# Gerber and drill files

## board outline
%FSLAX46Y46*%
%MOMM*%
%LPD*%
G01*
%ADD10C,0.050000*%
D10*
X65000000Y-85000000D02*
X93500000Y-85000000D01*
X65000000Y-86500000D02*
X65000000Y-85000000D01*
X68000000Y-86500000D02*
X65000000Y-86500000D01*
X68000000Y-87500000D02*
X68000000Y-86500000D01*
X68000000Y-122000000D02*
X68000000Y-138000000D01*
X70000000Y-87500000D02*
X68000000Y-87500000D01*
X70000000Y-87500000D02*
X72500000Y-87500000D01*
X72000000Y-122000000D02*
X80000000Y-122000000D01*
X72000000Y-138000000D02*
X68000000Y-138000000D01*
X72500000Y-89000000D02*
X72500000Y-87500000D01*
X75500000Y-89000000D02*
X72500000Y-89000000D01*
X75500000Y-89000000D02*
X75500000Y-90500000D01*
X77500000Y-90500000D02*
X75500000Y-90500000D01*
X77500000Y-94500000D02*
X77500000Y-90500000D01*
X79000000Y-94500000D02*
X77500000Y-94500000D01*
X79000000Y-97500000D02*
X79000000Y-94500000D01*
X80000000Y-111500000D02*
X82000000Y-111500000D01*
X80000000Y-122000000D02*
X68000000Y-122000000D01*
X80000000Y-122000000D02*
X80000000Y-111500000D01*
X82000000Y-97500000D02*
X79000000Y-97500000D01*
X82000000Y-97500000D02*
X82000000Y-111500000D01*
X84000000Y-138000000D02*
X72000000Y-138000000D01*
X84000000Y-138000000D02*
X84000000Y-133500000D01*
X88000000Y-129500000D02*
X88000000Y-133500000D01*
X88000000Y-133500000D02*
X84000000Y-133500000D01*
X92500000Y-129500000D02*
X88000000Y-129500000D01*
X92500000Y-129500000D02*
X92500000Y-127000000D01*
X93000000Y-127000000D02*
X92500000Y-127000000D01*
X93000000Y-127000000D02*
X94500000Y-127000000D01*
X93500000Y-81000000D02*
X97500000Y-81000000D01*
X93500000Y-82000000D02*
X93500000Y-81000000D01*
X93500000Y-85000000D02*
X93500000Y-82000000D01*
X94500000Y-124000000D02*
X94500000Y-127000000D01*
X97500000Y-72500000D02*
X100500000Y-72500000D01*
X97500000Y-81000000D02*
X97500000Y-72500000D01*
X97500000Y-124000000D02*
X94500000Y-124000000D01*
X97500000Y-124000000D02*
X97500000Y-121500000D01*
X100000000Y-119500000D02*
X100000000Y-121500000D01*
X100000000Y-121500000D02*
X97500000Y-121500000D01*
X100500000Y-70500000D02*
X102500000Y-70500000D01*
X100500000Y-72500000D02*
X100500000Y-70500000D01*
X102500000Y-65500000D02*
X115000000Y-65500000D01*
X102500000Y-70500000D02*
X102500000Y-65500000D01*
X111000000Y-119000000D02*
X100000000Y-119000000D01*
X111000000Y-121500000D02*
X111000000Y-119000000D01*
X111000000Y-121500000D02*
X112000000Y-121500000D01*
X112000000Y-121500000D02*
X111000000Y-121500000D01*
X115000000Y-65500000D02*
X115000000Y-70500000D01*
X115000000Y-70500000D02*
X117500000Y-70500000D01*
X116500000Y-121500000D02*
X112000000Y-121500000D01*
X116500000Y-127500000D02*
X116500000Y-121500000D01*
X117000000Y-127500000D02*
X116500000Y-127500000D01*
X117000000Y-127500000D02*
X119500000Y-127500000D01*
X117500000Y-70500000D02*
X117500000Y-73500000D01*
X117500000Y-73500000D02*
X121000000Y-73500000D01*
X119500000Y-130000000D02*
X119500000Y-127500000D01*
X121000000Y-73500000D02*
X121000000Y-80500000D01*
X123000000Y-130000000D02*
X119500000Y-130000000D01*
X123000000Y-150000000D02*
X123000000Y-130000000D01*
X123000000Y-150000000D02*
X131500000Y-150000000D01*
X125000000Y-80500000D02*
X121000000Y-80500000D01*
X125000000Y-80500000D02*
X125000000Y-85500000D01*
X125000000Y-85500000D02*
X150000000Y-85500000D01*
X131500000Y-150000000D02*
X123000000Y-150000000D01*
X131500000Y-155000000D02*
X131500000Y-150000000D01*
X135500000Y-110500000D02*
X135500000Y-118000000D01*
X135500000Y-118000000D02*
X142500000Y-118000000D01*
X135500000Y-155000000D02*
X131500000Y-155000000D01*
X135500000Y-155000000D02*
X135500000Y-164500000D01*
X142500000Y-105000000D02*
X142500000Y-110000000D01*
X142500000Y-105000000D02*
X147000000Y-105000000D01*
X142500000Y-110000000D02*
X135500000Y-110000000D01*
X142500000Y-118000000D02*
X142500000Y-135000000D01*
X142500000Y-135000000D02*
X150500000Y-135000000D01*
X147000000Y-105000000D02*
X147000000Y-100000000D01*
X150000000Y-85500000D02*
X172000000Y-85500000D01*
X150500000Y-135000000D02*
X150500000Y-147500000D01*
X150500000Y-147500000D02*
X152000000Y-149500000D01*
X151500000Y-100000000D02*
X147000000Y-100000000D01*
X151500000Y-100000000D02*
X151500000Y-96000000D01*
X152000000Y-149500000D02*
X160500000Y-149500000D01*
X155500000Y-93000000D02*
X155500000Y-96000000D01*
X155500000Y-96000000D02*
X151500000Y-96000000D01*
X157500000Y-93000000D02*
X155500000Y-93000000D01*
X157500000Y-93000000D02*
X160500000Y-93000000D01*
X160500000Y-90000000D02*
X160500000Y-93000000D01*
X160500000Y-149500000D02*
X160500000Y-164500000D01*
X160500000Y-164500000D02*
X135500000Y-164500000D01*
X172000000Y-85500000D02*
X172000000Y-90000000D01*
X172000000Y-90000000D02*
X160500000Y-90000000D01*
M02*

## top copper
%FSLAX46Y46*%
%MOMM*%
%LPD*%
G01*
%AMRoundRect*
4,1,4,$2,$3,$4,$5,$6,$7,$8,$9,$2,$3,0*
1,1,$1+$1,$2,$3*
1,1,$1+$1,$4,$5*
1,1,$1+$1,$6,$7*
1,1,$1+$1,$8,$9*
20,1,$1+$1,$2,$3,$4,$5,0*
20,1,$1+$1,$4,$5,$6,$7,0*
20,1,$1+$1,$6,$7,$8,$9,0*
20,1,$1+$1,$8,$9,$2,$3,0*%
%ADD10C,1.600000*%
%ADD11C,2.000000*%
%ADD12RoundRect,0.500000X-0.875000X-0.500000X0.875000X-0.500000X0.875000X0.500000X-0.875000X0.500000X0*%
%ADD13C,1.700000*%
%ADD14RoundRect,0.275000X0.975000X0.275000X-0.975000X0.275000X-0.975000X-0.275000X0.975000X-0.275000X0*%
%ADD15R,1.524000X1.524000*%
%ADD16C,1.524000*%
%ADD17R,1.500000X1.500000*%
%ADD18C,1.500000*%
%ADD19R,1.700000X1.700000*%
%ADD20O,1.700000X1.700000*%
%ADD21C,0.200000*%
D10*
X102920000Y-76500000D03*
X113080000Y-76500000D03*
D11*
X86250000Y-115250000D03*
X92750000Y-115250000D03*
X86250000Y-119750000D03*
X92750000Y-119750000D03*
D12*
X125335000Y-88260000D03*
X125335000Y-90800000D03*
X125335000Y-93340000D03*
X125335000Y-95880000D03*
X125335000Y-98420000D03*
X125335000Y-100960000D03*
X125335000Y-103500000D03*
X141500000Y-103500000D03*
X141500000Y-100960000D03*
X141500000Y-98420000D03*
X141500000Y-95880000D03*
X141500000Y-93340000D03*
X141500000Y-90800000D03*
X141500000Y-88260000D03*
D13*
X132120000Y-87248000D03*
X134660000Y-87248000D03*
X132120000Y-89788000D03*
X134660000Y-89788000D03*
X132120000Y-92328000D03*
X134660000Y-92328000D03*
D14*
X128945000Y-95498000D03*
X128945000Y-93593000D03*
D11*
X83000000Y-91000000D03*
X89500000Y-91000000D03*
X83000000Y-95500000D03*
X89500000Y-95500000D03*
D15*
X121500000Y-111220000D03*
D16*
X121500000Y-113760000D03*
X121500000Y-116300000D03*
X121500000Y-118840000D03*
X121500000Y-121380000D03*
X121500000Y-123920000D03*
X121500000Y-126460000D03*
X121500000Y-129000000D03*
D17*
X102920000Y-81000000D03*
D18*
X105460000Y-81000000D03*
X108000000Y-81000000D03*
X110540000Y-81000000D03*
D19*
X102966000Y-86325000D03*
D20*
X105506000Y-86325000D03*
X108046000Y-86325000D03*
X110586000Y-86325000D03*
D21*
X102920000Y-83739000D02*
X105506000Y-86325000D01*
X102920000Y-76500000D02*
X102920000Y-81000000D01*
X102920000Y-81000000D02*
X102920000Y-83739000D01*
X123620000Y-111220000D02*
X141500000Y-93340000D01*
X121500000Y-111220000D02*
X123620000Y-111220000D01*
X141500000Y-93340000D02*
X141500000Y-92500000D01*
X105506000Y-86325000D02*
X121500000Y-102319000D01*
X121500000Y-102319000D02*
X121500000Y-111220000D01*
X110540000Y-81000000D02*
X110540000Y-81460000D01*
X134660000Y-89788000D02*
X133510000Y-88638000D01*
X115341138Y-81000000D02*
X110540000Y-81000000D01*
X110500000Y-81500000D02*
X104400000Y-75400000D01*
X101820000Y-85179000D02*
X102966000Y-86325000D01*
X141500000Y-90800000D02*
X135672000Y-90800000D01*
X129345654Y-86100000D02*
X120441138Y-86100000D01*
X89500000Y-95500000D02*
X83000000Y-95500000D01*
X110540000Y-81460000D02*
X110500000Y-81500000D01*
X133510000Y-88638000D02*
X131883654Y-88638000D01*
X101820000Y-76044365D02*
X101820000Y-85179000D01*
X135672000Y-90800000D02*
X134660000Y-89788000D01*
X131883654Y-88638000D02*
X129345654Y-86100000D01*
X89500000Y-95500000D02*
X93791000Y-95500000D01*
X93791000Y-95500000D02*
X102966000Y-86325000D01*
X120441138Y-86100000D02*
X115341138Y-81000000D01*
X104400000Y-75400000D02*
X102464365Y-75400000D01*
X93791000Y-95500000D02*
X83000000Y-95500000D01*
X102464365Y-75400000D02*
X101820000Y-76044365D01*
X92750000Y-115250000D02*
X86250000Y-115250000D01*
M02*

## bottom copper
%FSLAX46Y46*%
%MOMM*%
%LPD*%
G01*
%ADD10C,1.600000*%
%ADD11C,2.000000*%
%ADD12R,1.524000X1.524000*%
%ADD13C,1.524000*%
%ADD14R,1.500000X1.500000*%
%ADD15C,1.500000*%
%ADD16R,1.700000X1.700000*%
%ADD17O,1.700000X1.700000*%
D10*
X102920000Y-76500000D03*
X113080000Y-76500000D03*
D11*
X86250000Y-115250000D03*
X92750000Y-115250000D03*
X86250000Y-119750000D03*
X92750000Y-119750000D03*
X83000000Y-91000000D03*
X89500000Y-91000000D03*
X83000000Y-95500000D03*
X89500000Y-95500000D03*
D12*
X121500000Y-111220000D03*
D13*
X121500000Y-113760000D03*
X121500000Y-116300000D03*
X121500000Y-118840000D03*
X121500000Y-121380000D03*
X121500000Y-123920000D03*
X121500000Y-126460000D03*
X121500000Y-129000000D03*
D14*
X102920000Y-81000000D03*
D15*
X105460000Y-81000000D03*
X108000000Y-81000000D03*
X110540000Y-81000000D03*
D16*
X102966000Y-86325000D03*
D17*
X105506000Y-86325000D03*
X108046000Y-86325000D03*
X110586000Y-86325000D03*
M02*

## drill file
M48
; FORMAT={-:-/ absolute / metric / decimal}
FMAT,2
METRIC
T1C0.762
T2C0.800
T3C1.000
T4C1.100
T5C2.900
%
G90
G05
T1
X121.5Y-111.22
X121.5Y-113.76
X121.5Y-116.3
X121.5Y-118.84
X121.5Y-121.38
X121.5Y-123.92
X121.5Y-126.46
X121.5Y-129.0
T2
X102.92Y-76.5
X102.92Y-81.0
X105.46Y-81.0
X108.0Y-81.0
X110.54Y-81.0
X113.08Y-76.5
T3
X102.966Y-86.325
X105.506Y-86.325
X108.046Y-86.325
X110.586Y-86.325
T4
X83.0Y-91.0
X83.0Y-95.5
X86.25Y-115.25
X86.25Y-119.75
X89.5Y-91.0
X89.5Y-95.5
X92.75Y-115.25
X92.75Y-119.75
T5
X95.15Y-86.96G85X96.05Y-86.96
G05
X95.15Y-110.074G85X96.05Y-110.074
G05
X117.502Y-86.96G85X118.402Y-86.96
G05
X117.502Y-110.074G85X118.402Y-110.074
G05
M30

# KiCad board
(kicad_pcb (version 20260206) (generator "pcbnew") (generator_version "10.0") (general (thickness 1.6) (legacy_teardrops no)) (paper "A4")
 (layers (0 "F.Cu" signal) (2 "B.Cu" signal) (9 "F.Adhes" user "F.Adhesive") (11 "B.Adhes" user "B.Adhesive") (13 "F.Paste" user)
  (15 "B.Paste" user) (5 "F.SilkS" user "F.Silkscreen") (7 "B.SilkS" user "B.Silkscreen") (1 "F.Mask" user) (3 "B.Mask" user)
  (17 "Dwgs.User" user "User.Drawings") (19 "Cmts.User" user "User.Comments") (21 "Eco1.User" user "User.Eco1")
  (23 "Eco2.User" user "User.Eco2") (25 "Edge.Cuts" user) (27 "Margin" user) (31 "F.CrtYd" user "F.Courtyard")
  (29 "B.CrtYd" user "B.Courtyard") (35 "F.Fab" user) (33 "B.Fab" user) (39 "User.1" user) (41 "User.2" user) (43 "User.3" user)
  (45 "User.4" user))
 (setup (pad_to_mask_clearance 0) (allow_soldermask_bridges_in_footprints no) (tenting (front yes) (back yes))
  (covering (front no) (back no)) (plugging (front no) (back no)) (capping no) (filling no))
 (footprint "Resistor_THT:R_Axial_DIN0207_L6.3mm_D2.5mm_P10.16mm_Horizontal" (layer "F.Cu") (at 102.92 76.5)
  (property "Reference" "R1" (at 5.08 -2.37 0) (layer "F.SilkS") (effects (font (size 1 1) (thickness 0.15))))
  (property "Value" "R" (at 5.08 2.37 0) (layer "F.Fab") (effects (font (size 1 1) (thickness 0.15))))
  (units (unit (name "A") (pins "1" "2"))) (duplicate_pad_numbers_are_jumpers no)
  (pad "1" thru_hole circle (at 0 0) (size 1.6 1.6) (drill 0.8) (layers "*.Cu" "*.Mask") (remove_unused_layers no) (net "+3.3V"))
  (pad "2" thru_hole circle (at 10.16 0) (size 1.6 1.6) (drill 0.8) (layers "*.Cu" "*.Mask") (remove_unused_layers no)
   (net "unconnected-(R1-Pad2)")))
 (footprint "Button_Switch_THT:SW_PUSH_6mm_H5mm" (layer "F.Cu") (at 86.25 115.25)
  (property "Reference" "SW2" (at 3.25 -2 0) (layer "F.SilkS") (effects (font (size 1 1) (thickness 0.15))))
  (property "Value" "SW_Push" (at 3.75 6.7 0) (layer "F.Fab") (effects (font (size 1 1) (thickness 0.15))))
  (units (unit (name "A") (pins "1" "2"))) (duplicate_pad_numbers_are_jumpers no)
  (pad "1" thru_hole circle (at 0 0 90) (size 2 2) (drill 1.1) (layers "*.Cu" "*.Mask") (remove_unused_layers no)
   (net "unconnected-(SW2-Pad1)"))
  (pad "1" thru_hole circle (at 6.5 0 90) (size 2 2) (drill 1.1) (layers "*.Cu" "*.Mask") (remove_unused_layers no)
   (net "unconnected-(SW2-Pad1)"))
  (pad "2" thru_hole circle (at 0 4.5 90) (size 2 2) (drill 1.1) (layers "*.Cu" "*.Mask") (remove_unused_layers no) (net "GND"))
  (pad "2" thru_hole circle (at 6.5 4.5 90) (size 2 2) (drill 1.1) (layers "*.Cu" "*.Mask") (remove_unused_layers no) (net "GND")))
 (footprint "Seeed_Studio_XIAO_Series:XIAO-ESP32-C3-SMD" (layer "F.Cu") (at 124.5 106.38)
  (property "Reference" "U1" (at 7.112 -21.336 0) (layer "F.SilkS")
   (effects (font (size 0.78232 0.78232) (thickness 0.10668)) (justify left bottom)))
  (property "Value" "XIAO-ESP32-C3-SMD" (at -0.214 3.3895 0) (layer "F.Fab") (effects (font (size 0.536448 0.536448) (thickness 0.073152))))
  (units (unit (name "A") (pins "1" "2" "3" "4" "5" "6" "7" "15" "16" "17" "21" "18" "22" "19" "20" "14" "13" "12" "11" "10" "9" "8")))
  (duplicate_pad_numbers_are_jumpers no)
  (pad "1" smd roundrect (at 0.835 -18.12) (size 2.75 2) (layers "F.Cu" "F.Mask" "F.Paste") (roundrect_rratio 0.25)
   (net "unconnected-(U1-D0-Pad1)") (solder_mask_margin 0.0508) (thermal_bridge_angle 45))
  (pad "2" smd roundrect (at 0.835 -15.58) (size 2.75 2) (layers "F.Cu" "F.Mask" "F.Paste") (roundrect_rratio 0.25)
   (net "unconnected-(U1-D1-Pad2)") (solder_mask_margin 0.0508) (thermal_bridge_angle 45))
  (pad "3" smd roundrect (at 0.835 -13.04) (size 2.75 2) (layers "F.Cu" "F.Mask" "F.Paste") (roundrect_rratio 0.25)
   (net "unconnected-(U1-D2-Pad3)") (solder_mask_margin 0.0508) (thermal_bridge_angle 45))
  (pad "4" smd roundrect (at 0.835 -10.5) (size 2.75 2) (layers "F.Cu" "F.Mask" "F.Paste") (roundrect_rratio 0.25)
   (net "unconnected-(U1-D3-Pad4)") (solder_mask_margin 0.0508) (thermal_bridge_angle 45))
  (pad "5" smd roundrect (at 0.835 -7.96) (size 2.75 2) (layers "F.Cu" "F.Mask" "F.Paste") (roundrect_rratio 0.25)
   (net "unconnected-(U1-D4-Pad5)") (solder_mask_margin 0.0508) (thermal_bridge_angle 45))
  (pad "6" smd roundrect (at 0.835 -5.42) (size 2.75 2) (layers "F.Cu" "F.Mask" "F.Paste") (roundrect_rratio 0.25)
   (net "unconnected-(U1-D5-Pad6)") (solder_mask_margin 0.0508) (thermal_bridge_angle 45))
  (pad "7" smd roundrect (at 0.835 -2.88) (size 2.75 2) (layers "F.Cu" "F.Mask" "F.Paste") (roundrect_rratio 0.25)
   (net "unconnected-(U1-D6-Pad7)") (solder_mask_margin 0.0508) (thermal_bridge_angle 45))
  (pad "8" smd roundrect (at 17 -2.88) (size 2.75 2) (layers "F.Cu" "F.Mask" "F.Paste") (roundrect_rratio 0.25)
   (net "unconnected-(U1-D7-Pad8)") (solder_mask_margin 0.0508) (thermal_bridge_angle 45))
  (pad "9" smd roundrect (at 17 -5.42) (size 2.75 2) (layers "F.Cu" "F.Mask" "F.Paste") (roundrect_rratio 0.25)
   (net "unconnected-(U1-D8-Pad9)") (solder_mask_margin 0.0508) (thermal_bridge_angle 45))
  (pad "10" smd roundrect (at 17 -7.96) (size 2.75 2) (layers "F.Cu" "F.Mask" "F.Paste") (roundrect_rratio 0.25)
   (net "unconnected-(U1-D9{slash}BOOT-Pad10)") (solder_mask_margin 0.0508) (thermal_bridge_angle 45))
  (pad "11" smd roundrect (at 17 -10.5) (size 2.75 2) (layers "F.Cu" "F.Mask" "F.Paste") (roundrect_rratio 0.25)
   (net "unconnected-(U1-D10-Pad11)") (solder_mask_margin 0.0508) (thermal_bridge_angle 45))
  (pad "12" smd roundrect (at 17 -13.04) (size 2.75 2) (layers "F.Cu" "F.Mask" "F.Paste") (roundrect_rratio 0.25) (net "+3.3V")
   (solder_mask_margin 0.0508) (thermal_bridge_angle 45))
  (pad "13" smd roundrect (at 17 -15.58) (size 2.75 2) (layers "F.Cu" "F.Mask" "F.Paste") (roundrect_rratio 0.25) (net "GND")
   (solder_mask_margin 0.0508) (thermal_bridge_angle 45))
  (pad "14" smd roundrect (at 17 -18.12) (size 2.75 2) (layers "F.Cu" "F.Mask" "F.Paste") (roundrect_rratio 0.25) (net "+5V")
   (solder_mask_margin 0.0508) (thermal_bridge_angle 45))
  (pad "15" smd circle (at 7.62 -19.132) (size 1.7 1.7) (layers "F.Cu" "F.Mask" "F.Paste") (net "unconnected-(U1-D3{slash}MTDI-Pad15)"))
  (pad "16" smd circle (at 10.16 -19.132) (size 1.7 1.7) (layers "F.Cu" "F.Mask" "F.Paste") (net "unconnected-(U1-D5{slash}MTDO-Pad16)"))
  (pad "17" smd circle (at 7.62 -16.592) (size 1.7 1.7) (layers "F.Cu" "F.Mask" "F.Paste") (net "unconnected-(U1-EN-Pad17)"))
  (pad "18" smd circle (at 10.16 -16.592) (size 1.7 1.7) (layers "F.Cu" "F.Mask" "F.Paste") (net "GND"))
  (pad "19" smd circle (at 7.62 -14.052) (size 1.7 1.7) (layers "F.Cu" "F.Mask" "F.Paste") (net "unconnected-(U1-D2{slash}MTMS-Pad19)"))
  (pad "20" smd circle (at 10.16 -14.052) (size 1.7 1.7) (layers "F.Cu" "F.Mask" "F.Paste") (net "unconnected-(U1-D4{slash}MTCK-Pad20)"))
  (pad "21" smd roundrect (at 4.445 -10.882 180) (size 2.5 1.1) (layers "F.Cu" "F.Mask" "F.Paste") (roundrect_rratio 0.25)
   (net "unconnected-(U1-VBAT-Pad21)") (thermal_bridge_angle 45))
  (pad "22" smd roundrect (at 4.445 -12.787 180) (size 2.5 1.1) (layers "F.Cu" "F.Mask" "F.Paste") (roundrect_rratio 0.25)
   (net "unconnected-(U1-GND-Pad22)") (thermal_bridge_angle 45)))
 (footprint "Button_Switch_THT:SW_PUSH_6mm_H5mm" (layer "F.Cu") (at 83 91)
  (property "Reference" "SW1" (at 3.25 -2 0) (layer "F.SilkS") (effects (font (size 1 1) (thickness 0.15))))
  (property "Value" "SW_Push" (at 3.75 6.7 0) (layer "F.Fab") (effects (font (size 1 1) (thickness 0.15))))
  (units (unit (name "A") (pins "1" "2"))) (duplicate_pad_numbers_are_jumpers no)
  (pad "1" thru_hole circle (at 0 0 90) (size 2 2) (drill 1.1) (layers "*.Cu" "*.Mask") (remove_unused_layers no)
   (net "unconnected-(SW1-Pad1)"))
  (pad "1" thru_hole circle (at 6.5 0 90) (size 2 2) (drill 1.1) (layers "*.Cu" "*.Mask") (remove_unused_layers no)
   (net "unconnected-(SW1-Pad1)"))
  (pad "2" thru_hole circle (at 0 4.5 90) (size 2 2) (drill 1.1) (layers "*.Cu" "*.Mask") (remove_unused_layers no) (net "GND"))
  (pad "2" thru_hole circle (at 6.5 4.5 90) (size 2 2) (drill 1.1) (layers "*.Cu" "*.Mask") (remove_unused_layers no) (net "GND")))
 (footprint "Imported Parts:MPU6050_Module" (layer "F.Cu") (at 121.5 111.22)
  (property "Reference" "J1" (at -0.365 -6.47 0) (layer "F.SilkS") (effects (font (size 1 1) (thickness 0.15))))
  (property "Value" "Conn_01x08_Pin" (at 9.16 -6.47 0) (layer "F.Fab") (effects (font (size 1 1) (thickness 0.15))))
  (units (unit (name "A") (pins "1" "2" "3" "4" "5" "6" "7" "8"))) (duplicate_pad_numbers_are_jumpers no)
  (pad "1" thru_hole rect (at 0 0) (size 1.524 1.524) (drill 0.762) (layers "*.Cu" "*.Mask") (remove_unused_layers no) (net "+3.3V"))
  (pad "2" thru_hole circle (at 0 2.54) (size 1.524 1.524) (drill 0.762) (layers "*.Cu" "*.Mask") (remove_unused_layers no) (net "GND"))
  (pad "3" thru_hole circle (at 0 5.08) (size 1.524 1.524) (drill 0.762) (layers "*.Cu" "*.Mask") (remove_unused_layers no) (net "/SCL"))
  (pad "4" thru_hole circle (at 0 7.62) (size 1.524 1.524) (drill 0.762) (layers "*.Cu" "*.Mask") (remove_unused_layers no) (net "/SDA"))
  (pad "5" thru_hole circle (at 0 10.16) (size 1.524 1.524) (drill 0.762) (layers "*.Cu" "*.Mask") (remove_unused_layers no)
   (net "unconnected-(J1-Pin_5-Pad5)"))
  (pad "6" thru_hole circle (at 0 12.7) (size 1.524 1.524) (drill 0.762) (layers "*.Cu" "*.Mask") (remove_unused_layers no)
   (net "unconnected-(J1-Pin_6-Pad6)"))
  (pad "7" thru_hole circle (at 0 15.24) (size 1.524 1.524) (drill 0.762) (layers "*.Cu" "*.Mask") (remove_unused_layers no)
   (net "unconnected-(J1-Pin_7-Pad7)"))
  (pad "8" thru_hole circle (at 0 17.78) (size 1.524 1.524) (drill 0.762) (layers "*.Cu" "*.Mask") (remove_unused_layers no)
   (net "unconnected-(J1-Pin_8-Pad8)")))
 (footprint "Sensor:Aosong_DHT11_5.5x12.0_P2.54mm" (layer "F.Cu") (at 102.92 81 90)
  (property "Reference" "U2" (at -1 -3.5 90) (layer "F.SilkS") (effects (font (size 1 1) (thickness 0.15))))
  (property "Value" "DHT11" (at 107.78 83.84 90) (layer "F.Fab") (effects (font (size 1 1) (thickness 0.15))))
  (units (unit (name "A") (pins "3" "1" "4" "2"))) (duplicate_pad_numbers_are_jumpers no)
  (pad "1" thru_hole rect (at 0 0 90) (size 1.5 1.5) (drill 0.8) (layers "*.Cu" "*.Mask") (remove_unused_layers no) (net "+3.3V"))
  (pad "2" thru_hole circle (at 0 2.54 90) (size 1.5 1.5) (drill 0.8) (layers "*.Cu" "*.Mask") (remove_unused_layers no)
   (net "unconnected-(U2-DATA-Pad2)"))
  (pad "3" thru_hole circle (at 0 5.08 90) (size 1.5 1.5) (drill 0.8) (layers "*.Cu" "*.Mask") (remove_unused_layers no)
   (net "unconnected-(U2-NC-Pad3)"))
  (pad "4" thru_hole circle (at 0 7.62 90) (size 1.5 1.5) (drill 0.8) (layers "*.Cu" "*.Mask") (remove_unused_layers no) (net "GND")))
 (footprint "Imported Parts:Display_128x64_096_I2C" (layer "F.Cu") (at 106.776 86.325)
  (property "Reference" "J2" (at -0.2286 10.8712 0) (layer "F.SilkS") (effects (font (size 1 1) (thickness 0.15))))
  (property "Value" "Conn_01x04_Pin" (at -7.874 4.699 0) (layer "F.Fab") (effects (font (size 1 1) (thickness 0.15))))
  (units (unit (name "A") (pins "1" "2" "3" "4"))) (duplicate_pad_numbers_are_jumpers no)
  (pad "" np_thru_hole oval (at -11.176 0.635) (size 3.8 2.9) (drill oval 3.8 2.9) (layers "*.Cu" "*.Mask"))
  (pad "" np_thru_hole oval (at -11.176 23.749) (size 3.8 2.9) (drill oval 3.8 2.9) (layers "*.Cu" "*.Mask"))
  (pad "" np_thru_hole oval (at 11.176 0.635) (size 3.8 2.9) (drill oval 3.8 2.9) (layers "*.Cu" "*.Mask"))
  (pad "" np_thru_hole oval (at 11.176 23.749) (size 3.8 2.9) (drill oval 3.8 2.9) (layers "*.Cu" "*.Mask"))
  (pad "1" thru_hole rect (at -3.81 0 90) (size 1.7 1.7) (drill 1) (layers "*.Cu" "*.Mask") (remove_unused_layers no) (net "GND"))
  (pad "2" thru_hole oval (at -1.27 0 90) (size 1.7 1.7) (drill 1) (layers "*.Cu" "*.Mask") (remove_unused_layers no) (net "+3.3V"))
  (pad "3" thru_hole oval (at 1.27 0 90) (size 1.7 1.7) (drill 1) (layers "*.Cu" "*.Mask") (remove_unused_layers no)
   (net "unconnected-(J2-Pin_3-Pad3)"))
  (pad "4" thru_hole oval (at 3.81 0 90) (size 1.7 1.7) (drill 1) (layers "*.Cu" "*.Mask") (remove_unused_layers no)
   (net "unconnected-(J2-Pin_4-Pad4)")))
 (gr_line (start 65 85) (end 93.5 85) (stroke (width 0.05) (type default)) (layer "Edge.Cuts"))
 (gr_line (start 65 86.5) (end 65 85) (stroke (width 0.05) (type default)) (layer "Edge.Cuts"))
 (gr_line (start 68 86.5) (end 65 86.5) (stroke (width 0.05) (type default)) (layer "Edge.Cuts"))
 (gr_line (start 68 87.5) (end 68 86.5) (stroke (width 0.05) (type default)) (layer "Edge.Cuts"))
 (gr_line (start 68 122) (end 68 138) (stroke (width 0.05) (type default)) (layer "Edge.Cuts"))
 (gr_line (start 70 87.5) (end 68 87.5) (stroke (width 0.05) (type default)) (layer "Edge.Cuts"))
 (gr_line (start 70 87.5) (end 72.5 87.5) (stroke (width 0.05) (type default)) (layer "Edge.Cuts"))
 (gr_line (start 72 122) (end 80 122) (stroke (width 0.05) (type default)) (layer "Edge.Cuts"))
 (gr_line (start 72 138) (end 68 138) (stroke (width 0.05) (type default)) (layer "Edge.Cuts"))
 (gr_line (start 72.5 89) (end 72.5 87.5) (stroke (width 0.05) (type default)) (layer "Edge.Cuts"))
 (gr_line (start 75.5 89) (end 72.5 89) (stroke (width 0.05) (type default)) (layer "Edge.Cuts"))
 (gr_line (start 75.5 89) (end 75.5 90.5) (stroke (width 0.05) (type default)) (layer "Edge.Cuts"))
 (gr_line (start 77.5 90.5) (end 75.5 90.5) (stroke (width 0.05) (type default)) (layer "Edge.Cuts"))
 (gr_line (start 77.5 94.5) (end 77.5 90.5) (stroke (width 0.05) (type default)) (layer "Edge.Cuts"))
 (gr_line (start 79 94.5) (end 77.5 94.5) (stroke (width 0.05) (type default)) (layer "Edge.Cuts"))
 (gr_line (start 79 97.5) (end 79 94.5) (stroke (width 0.05) (type default)) (layer "Edge.Cuts"))
 (gr_line (start 80 111.5) (end 82 111.5) (stroke (width 0.05) (type default)) (layer "Edge.Cuts"))
 (gr_line (start 80 122) (end 68 122) (stroke (width 0.05) (type default)) (layer "Edge.Cuts"))
 (gr_line (start 80 122) (end 80 111.5) (stroke (width 0.05) (type default)) (layer "Edge.Cuts"))
 (gr_line (start 82 97.5) (end 79 97.5) (stroke (width 0.05) (type default)) (layer "Edge.Cuts"))
 (gr_line (start 82 97.5) (end 82 111.5) (stroke (width 0.05) (type default)) (layer "Edge.Cuts"))
 (gr_line (start 84 138) (end 72 138) (stroke (width 0.05) (type default)) (layer "Edge.Cuts"))
 (gr_line (start 84 138) (end 84 133.5) (stroke (width 0.05) (type default)) (layer "Edge.Cuts"))
 (gr_line (start 88 129.5) (end 88 133.5) (stroke (width 0.05) (type default)) (layer "Edge.Cuts"))
 (gr_line (start 88 133.5) (end 84 133.5) (stroke (width 0.05) (type default)) (layer "Edge.Cuts"))
 (gr_line (start 92.5 129.5) (end 88 129.5) (stroke (width 0.05) (type default)) (layer "Edge.Cuts"))
 (gr_line (start 92.5 129.5) (end 92.5 127) (stroke (width 0.05) (type default)) (layer "Edge.Cuts"))
 (gr_line (start 93 127) (end 92.5 127) (stroke (width 0.05) (type default)) (layer "Edge.Cuts"))
 (gr_line (start 93 127) (end 94.5 127) (stroke (width 0.05) (type default)) (layer "Edge.Cuts"))
 (gr_line (start 93.5 81) (end 97.5 81) (stroke (width 0.05) (type default)) (layer "Edge.Cuts"))
 (gr_line (start 93.5 82) (end 93.5 81) (stroke (width 0.05) (type default)) (layer "Edge.Cuts"))
 (gr_line (start 93.5 85) (end 93.5 82) (stroke (width 0.05) (type default)) (layer "Edge.Cuts"))
 (gr_line (start 94.5 124) (end 94.5 127) (stroke (width 0.05) (type default)) (layer "Edge.Cuts"))
 (gr_line (start 97.5 72.5) (end 100.5 72.5) (stroke (width 0.05) (type default)) (layer "Edge.Cuts"))
 (gr_line (start 97.5 81) (end 97.5 72.5) (stroke (width 0.05) (type default)) (layer "Edge.Cuts"))
 (gr_line (start 97.5 124) (end 94.5 124) (stroke (width 0.05) (type default)) (layer "Edge.Cuts"))
 (gr_line (start 97.5 124) (end 97.5 121.5) (stroke (width 0.05) (type default)) (layer "Edge.Cuts"))
 (gr_line (start 100 119.5) (end 100 121.5) (stroke (width 0.05) (type default)) (layer "Edge.Cuts"))
 (gr_line (start 100 121.5) (end 97.5 121.5) (stroke (width 0.05) (type default)) (layer "Edge.Cuts"))
 (gr_line (start 100.5 70.5) (end 102.5 70.5) (stroke (width 0.05) (type default)) (layer "Edge.Cuts"))
 (gr_line (start 100.5 72.5) (end 100.5 70.5) (stroke (width 0.05) (type default)) (layer "Edge.Cuts"))
 (gr_line (start 102.5 65.5) (end 115 65.5) (stroke (width 0.05) (type default)) (layer "Edge.Cuts"))
 (gr_line (start 102.5 70.5) (end 102.5 65.5) (stroke (width 0.05) (type default)) (layer "Edge.Cuts"))
 (gr_line (start 111 119) (end 100 119) (stroke (width 0.05) (type default)) (layer "Edge.Cuts"))
 (gr_line (start 111 121.5) (end 111 119) (stroke (width 0.05) (type default)) (layer "Edge.Cuts"))
 (gr_line (start 111 121.5) (end 112 121.5) (stroke (width 0.05) (type default)) (layer "Edge.Cuts"))
 (gr_line (start 112 121.5) (end 111 121.5) (stroke (width 0.05) (type default)) (layer "Edge.Cuts"))
 (gr_line (start 115 65.5) (end 115 70.5) (stroke (width 0.05) (type default)) (layer "Edge.Cuts"))
 (gr_line (start 115 70.5) (end 117.5 70.5) (stroke (width 0.05) (type default)) (layer "Edge.Cuts"))
 (gr_line (start 116.5 121.5) (end 112 121.5) (stroke (width 0.05) (type default)) (layer "Edge.Cuts"))
 (gr_line (start 116.5 127.5) (end 116.5 121.5) (stroke (width 0.05) (type default)) (layer "Edge.Cuts"))
 (gr_line (start 117 127.5) (end 116.5 127.5) (stroke (width 0.05) (type default)) (layer "Edge.Cuts"))
 (gr_line (start 117 127.5) (end 119.5 127.5) (stroke (width 0.05) (type default)) (layer "Edge.Cuts"))
 (gr_line (start 117.5 70.5) (end 117.5 73.5) (stroke (width 0.05) (type default)) (layer "Edge.Cuts"))
 (gr_line (start 117.5 73.5) (end 121 73.5) (stroke (width 0.05) (type default)) (layer "Edge.Cuts"))
 (gr_line (start 119.5 130) (end 119.5 127.5) (stroke (width 0.05) (type default)) (layer "Edge.Cuts"))
 (gr_line (start 121 73.5) (end 121 80.5) (stroke (width 0.05) (type default)) (layer "Edge.Cuts"))
 (gr_line (start 123 130) (end 119.5 130) (stroke (width 0.05) (type default)) (layer "Edge.Cuts"))
 (gr_line (start 123 150) (end 123 130) (stroke (width 0.05) (type default)) (layer "Edge.Cuts"))
 (gr_line (start 123 150) (end 131.5 150) (stroke (width 0.05) (type default)) (layer "Edge.Cuts"))
 (gr_line (start 125 80.5) (end 121 80.5) (stroke (width 0.05) (type default)) (layer "Edge.Cuts"))
 (gr_line (start 125 80.5) (end 125 85.5) (stroke (width 0.05) (type default)) (layer "Edge.Cuts"))
 (gr_line (start 125 85.5) (end 150 85.5) (stroke (width 0.05) (type default)) (layer "Edge.Cuts"))
 (gr_line (start 131.5 150) (end 123 150) (stroke (width 0.05) (type default)) (layer "Edge.Cuts"))
 (gr_line (start 131.5 155) (end 131.5 150) (stroke (width 0.05) (type default)) (layer "Edge.Cuts"))
 (gr_line (start 135.5 110.5) (end 135.5 118) (stroke (width 0.05) (type default)) (layer "Edge.Cuts"))
 (gr_line (start 135.5 118) (end 142.5 118) (stroke (width 0.05) (type default)) (layer "Edge.Cuts"))
 (gr_line (start 135.5 155) (end 131.5 155) (stroke (width 0.05) (type default)) (layer "Edge.Cuts"))
 (gr_line (start 135.5 155) (end 135.5 164.5) (stroke (width 0.05) (type default)) (layer "Edge.Cuts"))
 (gr_line (start 142.5 105) (end 142.5 110) (stroke (width 0.05) (type default)) (layer "Edge.Cuts"))
 (gr_line (start 142.5 105) (end 147 105) (stroke (width 0.05) (type default)) (layer "Edge.Cuts"))
 (gr_line (start 142.5 110) (end 135.5 110) (stroke (width 0.05) (type default)) (layer "Edge.Cuts"))
 (gr_line (start 142.5 118) (end 142.5 135) (stroke (width 0.05) (type default)) (layer "Edge.Cuts"))
 (gr_line (start 142.5 135) (end 150.5 135) (stroke (width 0.05) (type default)) (layer "Edge.Cuts"))
 (gr_line (start 147 105) (end 147 100) (stroke (width 0.05) (type default)) (layer "Edge.Cuts"))
 (gr_line (start 150 85.5) (end 172 85.5) (stroke (width 0.05) (type default)) (layer "Edge.Cuts"))
 (gr_line (start 150.5 135) (end 150.5 147.5) (stroke (width 0.05) (type default)) (layer "Edge.Cuts"))
 (gr_line (start 150.5 147.5) (end 152 149.5) (stroke (width 0.05) (type default)) (layer "Edge.Cuts"))
 (gr_line (start 151.5 100) (end 147 100) (stroke (width 0.05) (type default)) (layer "Edge.Cuts"))
 (gr_line (start 151.5 100) (end 151.5 96) (stroke (width 0.05) (type default)) (layer "Edge.Cuts"))
 (gr_line (start 152 149.5) (end 160.5 149.5) (stroke (width 0.05) (type default)) (layer "Edge.Cuts"))
 (gr_line (start 155.5 93) (end 155.5 96) (stroke (width 0.05) (type default)) (layer "Edge.Cuts"))
 (gr_line (start 155.5 96) (end 151.5 96) (stroke (width 0.05) (type default)) (layer "Edge.Cuts"))
 (gr_line (start 157.5 93) (end 155.5 93) (stroke (width 0.05) (type default)) (layer "Edge.Cuts"))
 (gr_line (start 157.5 93) (end 160.5 93) (stroke (width 0.05) (type default)) (layer "Edge.Cuts"))
 (gr_line (start 160.5 90) (end 160.5 93) (stroke (width 0.05) (type default)) (layer "Edge.Cuts"))
 (gr_line (start 160.5 149.5) (end 160.5 164.5) (stroke (width 0.05) (type default)) (layer "Edge.Cuts"))
 (gr_line (start 160.5 164.5) (end 135.5 164.5) (stroke (width 0.05) (type default)) (layer "Edge.Cuts"))
 (gr_line (start 172 85.5) (end 172 90) (stroke (width 0.05) (type default)) (layer "Edge.Cuts"))
 (gr_line (start 172 90) (end 160.5 90) (stroke (width 0.05) (type default)) (layer "Edge.Cuts"))
 (segment (start 102.92 83.739) (end 105.506 86.325) (width 0.2) (layer "F.Cu") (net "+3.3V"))
 (segment (start 102.92 76.5) (end 102.92 81) (width 0.2) (layer "F.Cu") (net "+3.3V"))
 (segment (start 102.92 81) (end 102.92 83.739) (width 0.2) (layer "F.Cu") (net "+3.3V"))
 (segment (start 123.62 111.22) (end 141.5 93.34) (width 0.2) (layer "F.Cu") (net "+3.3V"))
 (segment (start 121.5 111.22) (end 123.62 111.22) (width 0.2) (layer "F.Cu") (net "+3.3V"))
 (segment (start 141.5 93.34) (end 141.5 92.5) (width 0.2) (layer "F.Cu") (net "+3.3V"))
 (segment (start 105.506 86.325) (end 121.5 102.319) (width 0.2) (layer "F.Cu") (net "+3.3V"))
 (segment (start 121.5 102.319) (end 121.5 111.22) (width 0.2) (layer "F.Cu") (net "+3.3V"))
 (segment (start 110.54 81) (end 110.54 81.46) (width 0.2) (layer "F.Cu") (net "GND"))
 (segment (start 134.66 89.788) (end 133.51 88.638) (width 0.2) (layer "F.Cu") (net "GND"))
 (segment (start 115.341138 81) (end 110.54 81) (width 0.2) (layer "F.Cu") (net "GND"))
 (segment (start 110.5 81.5) (end 104.4 75.4) (width 0.2) (layer "F.Cu") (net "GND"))
 (segment (start 101.82 85.179) (end 102.966 86.325) (width 0.2) (layer "F.Cu") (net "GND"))
 (segment (start 141.5 90.8) (end 135.672 90.8) (width 0.2) (layer "F.Cu") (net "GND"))
 (segment (start 129.345654 86.1) (end 120.441138 86.1) (width 0.2) (layer "F.Cu") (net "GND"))
 (segment (start 89.5 95.5) (end 83 95.5) (width 0.2) (layer "F.Cu") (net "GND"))
 (segment (start 110.54 81.46) (end 110.5 81.5) (width 0.2) (layer "F.Cu") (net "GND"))
 (segment (start 133.51 88.638) (end 131.883654 88.638) (width 0.2) (layer "F.Cu") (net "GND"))
 (segment (start 101.82 76.044365) (end 101.82 85.179) (width 0.2) (layer "F.Cu") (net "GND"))
 (segment (start 135.672 90.8) (end 134.66 89.788) (width 0.2) (layer "F.Cu") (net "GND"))
 (segment (start 131.883654 88.638) (end 129.345654 86.1) (width 0.2) (layer "F.Cu") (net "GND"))
 (segment (start 89.5 95.5) (end 93.791 95.5) (width 0.2) (layer "F.Cu") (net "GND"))
 (segment (start 93.791 95.5) (end 102.966 86.325) (width 0.2) (layer "F.Cu") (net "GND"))
 (segment (start 120.441138 86.1) (end 115.341138 81) (width 0.2) (layer "F.Cu") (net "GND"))
 (segment (start 104.4 75.4) (end 102.464365 75.4) (width 0.2) (layer "F.Cu") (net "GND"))
 (segment (start 93.791 95.5) (end 83 95.5) (width 0.2) (layer "F.Cu") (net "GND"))
 (segment (start 102.464365 75.4) (end 101.82 76.044365) (width 0.2) (layer "F.Cu") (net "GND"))
 (segment (start 92.75 115.25) (end 86.25 115.25) (width 0.2) (layer "F.Cu") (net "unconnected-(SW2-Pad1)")))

